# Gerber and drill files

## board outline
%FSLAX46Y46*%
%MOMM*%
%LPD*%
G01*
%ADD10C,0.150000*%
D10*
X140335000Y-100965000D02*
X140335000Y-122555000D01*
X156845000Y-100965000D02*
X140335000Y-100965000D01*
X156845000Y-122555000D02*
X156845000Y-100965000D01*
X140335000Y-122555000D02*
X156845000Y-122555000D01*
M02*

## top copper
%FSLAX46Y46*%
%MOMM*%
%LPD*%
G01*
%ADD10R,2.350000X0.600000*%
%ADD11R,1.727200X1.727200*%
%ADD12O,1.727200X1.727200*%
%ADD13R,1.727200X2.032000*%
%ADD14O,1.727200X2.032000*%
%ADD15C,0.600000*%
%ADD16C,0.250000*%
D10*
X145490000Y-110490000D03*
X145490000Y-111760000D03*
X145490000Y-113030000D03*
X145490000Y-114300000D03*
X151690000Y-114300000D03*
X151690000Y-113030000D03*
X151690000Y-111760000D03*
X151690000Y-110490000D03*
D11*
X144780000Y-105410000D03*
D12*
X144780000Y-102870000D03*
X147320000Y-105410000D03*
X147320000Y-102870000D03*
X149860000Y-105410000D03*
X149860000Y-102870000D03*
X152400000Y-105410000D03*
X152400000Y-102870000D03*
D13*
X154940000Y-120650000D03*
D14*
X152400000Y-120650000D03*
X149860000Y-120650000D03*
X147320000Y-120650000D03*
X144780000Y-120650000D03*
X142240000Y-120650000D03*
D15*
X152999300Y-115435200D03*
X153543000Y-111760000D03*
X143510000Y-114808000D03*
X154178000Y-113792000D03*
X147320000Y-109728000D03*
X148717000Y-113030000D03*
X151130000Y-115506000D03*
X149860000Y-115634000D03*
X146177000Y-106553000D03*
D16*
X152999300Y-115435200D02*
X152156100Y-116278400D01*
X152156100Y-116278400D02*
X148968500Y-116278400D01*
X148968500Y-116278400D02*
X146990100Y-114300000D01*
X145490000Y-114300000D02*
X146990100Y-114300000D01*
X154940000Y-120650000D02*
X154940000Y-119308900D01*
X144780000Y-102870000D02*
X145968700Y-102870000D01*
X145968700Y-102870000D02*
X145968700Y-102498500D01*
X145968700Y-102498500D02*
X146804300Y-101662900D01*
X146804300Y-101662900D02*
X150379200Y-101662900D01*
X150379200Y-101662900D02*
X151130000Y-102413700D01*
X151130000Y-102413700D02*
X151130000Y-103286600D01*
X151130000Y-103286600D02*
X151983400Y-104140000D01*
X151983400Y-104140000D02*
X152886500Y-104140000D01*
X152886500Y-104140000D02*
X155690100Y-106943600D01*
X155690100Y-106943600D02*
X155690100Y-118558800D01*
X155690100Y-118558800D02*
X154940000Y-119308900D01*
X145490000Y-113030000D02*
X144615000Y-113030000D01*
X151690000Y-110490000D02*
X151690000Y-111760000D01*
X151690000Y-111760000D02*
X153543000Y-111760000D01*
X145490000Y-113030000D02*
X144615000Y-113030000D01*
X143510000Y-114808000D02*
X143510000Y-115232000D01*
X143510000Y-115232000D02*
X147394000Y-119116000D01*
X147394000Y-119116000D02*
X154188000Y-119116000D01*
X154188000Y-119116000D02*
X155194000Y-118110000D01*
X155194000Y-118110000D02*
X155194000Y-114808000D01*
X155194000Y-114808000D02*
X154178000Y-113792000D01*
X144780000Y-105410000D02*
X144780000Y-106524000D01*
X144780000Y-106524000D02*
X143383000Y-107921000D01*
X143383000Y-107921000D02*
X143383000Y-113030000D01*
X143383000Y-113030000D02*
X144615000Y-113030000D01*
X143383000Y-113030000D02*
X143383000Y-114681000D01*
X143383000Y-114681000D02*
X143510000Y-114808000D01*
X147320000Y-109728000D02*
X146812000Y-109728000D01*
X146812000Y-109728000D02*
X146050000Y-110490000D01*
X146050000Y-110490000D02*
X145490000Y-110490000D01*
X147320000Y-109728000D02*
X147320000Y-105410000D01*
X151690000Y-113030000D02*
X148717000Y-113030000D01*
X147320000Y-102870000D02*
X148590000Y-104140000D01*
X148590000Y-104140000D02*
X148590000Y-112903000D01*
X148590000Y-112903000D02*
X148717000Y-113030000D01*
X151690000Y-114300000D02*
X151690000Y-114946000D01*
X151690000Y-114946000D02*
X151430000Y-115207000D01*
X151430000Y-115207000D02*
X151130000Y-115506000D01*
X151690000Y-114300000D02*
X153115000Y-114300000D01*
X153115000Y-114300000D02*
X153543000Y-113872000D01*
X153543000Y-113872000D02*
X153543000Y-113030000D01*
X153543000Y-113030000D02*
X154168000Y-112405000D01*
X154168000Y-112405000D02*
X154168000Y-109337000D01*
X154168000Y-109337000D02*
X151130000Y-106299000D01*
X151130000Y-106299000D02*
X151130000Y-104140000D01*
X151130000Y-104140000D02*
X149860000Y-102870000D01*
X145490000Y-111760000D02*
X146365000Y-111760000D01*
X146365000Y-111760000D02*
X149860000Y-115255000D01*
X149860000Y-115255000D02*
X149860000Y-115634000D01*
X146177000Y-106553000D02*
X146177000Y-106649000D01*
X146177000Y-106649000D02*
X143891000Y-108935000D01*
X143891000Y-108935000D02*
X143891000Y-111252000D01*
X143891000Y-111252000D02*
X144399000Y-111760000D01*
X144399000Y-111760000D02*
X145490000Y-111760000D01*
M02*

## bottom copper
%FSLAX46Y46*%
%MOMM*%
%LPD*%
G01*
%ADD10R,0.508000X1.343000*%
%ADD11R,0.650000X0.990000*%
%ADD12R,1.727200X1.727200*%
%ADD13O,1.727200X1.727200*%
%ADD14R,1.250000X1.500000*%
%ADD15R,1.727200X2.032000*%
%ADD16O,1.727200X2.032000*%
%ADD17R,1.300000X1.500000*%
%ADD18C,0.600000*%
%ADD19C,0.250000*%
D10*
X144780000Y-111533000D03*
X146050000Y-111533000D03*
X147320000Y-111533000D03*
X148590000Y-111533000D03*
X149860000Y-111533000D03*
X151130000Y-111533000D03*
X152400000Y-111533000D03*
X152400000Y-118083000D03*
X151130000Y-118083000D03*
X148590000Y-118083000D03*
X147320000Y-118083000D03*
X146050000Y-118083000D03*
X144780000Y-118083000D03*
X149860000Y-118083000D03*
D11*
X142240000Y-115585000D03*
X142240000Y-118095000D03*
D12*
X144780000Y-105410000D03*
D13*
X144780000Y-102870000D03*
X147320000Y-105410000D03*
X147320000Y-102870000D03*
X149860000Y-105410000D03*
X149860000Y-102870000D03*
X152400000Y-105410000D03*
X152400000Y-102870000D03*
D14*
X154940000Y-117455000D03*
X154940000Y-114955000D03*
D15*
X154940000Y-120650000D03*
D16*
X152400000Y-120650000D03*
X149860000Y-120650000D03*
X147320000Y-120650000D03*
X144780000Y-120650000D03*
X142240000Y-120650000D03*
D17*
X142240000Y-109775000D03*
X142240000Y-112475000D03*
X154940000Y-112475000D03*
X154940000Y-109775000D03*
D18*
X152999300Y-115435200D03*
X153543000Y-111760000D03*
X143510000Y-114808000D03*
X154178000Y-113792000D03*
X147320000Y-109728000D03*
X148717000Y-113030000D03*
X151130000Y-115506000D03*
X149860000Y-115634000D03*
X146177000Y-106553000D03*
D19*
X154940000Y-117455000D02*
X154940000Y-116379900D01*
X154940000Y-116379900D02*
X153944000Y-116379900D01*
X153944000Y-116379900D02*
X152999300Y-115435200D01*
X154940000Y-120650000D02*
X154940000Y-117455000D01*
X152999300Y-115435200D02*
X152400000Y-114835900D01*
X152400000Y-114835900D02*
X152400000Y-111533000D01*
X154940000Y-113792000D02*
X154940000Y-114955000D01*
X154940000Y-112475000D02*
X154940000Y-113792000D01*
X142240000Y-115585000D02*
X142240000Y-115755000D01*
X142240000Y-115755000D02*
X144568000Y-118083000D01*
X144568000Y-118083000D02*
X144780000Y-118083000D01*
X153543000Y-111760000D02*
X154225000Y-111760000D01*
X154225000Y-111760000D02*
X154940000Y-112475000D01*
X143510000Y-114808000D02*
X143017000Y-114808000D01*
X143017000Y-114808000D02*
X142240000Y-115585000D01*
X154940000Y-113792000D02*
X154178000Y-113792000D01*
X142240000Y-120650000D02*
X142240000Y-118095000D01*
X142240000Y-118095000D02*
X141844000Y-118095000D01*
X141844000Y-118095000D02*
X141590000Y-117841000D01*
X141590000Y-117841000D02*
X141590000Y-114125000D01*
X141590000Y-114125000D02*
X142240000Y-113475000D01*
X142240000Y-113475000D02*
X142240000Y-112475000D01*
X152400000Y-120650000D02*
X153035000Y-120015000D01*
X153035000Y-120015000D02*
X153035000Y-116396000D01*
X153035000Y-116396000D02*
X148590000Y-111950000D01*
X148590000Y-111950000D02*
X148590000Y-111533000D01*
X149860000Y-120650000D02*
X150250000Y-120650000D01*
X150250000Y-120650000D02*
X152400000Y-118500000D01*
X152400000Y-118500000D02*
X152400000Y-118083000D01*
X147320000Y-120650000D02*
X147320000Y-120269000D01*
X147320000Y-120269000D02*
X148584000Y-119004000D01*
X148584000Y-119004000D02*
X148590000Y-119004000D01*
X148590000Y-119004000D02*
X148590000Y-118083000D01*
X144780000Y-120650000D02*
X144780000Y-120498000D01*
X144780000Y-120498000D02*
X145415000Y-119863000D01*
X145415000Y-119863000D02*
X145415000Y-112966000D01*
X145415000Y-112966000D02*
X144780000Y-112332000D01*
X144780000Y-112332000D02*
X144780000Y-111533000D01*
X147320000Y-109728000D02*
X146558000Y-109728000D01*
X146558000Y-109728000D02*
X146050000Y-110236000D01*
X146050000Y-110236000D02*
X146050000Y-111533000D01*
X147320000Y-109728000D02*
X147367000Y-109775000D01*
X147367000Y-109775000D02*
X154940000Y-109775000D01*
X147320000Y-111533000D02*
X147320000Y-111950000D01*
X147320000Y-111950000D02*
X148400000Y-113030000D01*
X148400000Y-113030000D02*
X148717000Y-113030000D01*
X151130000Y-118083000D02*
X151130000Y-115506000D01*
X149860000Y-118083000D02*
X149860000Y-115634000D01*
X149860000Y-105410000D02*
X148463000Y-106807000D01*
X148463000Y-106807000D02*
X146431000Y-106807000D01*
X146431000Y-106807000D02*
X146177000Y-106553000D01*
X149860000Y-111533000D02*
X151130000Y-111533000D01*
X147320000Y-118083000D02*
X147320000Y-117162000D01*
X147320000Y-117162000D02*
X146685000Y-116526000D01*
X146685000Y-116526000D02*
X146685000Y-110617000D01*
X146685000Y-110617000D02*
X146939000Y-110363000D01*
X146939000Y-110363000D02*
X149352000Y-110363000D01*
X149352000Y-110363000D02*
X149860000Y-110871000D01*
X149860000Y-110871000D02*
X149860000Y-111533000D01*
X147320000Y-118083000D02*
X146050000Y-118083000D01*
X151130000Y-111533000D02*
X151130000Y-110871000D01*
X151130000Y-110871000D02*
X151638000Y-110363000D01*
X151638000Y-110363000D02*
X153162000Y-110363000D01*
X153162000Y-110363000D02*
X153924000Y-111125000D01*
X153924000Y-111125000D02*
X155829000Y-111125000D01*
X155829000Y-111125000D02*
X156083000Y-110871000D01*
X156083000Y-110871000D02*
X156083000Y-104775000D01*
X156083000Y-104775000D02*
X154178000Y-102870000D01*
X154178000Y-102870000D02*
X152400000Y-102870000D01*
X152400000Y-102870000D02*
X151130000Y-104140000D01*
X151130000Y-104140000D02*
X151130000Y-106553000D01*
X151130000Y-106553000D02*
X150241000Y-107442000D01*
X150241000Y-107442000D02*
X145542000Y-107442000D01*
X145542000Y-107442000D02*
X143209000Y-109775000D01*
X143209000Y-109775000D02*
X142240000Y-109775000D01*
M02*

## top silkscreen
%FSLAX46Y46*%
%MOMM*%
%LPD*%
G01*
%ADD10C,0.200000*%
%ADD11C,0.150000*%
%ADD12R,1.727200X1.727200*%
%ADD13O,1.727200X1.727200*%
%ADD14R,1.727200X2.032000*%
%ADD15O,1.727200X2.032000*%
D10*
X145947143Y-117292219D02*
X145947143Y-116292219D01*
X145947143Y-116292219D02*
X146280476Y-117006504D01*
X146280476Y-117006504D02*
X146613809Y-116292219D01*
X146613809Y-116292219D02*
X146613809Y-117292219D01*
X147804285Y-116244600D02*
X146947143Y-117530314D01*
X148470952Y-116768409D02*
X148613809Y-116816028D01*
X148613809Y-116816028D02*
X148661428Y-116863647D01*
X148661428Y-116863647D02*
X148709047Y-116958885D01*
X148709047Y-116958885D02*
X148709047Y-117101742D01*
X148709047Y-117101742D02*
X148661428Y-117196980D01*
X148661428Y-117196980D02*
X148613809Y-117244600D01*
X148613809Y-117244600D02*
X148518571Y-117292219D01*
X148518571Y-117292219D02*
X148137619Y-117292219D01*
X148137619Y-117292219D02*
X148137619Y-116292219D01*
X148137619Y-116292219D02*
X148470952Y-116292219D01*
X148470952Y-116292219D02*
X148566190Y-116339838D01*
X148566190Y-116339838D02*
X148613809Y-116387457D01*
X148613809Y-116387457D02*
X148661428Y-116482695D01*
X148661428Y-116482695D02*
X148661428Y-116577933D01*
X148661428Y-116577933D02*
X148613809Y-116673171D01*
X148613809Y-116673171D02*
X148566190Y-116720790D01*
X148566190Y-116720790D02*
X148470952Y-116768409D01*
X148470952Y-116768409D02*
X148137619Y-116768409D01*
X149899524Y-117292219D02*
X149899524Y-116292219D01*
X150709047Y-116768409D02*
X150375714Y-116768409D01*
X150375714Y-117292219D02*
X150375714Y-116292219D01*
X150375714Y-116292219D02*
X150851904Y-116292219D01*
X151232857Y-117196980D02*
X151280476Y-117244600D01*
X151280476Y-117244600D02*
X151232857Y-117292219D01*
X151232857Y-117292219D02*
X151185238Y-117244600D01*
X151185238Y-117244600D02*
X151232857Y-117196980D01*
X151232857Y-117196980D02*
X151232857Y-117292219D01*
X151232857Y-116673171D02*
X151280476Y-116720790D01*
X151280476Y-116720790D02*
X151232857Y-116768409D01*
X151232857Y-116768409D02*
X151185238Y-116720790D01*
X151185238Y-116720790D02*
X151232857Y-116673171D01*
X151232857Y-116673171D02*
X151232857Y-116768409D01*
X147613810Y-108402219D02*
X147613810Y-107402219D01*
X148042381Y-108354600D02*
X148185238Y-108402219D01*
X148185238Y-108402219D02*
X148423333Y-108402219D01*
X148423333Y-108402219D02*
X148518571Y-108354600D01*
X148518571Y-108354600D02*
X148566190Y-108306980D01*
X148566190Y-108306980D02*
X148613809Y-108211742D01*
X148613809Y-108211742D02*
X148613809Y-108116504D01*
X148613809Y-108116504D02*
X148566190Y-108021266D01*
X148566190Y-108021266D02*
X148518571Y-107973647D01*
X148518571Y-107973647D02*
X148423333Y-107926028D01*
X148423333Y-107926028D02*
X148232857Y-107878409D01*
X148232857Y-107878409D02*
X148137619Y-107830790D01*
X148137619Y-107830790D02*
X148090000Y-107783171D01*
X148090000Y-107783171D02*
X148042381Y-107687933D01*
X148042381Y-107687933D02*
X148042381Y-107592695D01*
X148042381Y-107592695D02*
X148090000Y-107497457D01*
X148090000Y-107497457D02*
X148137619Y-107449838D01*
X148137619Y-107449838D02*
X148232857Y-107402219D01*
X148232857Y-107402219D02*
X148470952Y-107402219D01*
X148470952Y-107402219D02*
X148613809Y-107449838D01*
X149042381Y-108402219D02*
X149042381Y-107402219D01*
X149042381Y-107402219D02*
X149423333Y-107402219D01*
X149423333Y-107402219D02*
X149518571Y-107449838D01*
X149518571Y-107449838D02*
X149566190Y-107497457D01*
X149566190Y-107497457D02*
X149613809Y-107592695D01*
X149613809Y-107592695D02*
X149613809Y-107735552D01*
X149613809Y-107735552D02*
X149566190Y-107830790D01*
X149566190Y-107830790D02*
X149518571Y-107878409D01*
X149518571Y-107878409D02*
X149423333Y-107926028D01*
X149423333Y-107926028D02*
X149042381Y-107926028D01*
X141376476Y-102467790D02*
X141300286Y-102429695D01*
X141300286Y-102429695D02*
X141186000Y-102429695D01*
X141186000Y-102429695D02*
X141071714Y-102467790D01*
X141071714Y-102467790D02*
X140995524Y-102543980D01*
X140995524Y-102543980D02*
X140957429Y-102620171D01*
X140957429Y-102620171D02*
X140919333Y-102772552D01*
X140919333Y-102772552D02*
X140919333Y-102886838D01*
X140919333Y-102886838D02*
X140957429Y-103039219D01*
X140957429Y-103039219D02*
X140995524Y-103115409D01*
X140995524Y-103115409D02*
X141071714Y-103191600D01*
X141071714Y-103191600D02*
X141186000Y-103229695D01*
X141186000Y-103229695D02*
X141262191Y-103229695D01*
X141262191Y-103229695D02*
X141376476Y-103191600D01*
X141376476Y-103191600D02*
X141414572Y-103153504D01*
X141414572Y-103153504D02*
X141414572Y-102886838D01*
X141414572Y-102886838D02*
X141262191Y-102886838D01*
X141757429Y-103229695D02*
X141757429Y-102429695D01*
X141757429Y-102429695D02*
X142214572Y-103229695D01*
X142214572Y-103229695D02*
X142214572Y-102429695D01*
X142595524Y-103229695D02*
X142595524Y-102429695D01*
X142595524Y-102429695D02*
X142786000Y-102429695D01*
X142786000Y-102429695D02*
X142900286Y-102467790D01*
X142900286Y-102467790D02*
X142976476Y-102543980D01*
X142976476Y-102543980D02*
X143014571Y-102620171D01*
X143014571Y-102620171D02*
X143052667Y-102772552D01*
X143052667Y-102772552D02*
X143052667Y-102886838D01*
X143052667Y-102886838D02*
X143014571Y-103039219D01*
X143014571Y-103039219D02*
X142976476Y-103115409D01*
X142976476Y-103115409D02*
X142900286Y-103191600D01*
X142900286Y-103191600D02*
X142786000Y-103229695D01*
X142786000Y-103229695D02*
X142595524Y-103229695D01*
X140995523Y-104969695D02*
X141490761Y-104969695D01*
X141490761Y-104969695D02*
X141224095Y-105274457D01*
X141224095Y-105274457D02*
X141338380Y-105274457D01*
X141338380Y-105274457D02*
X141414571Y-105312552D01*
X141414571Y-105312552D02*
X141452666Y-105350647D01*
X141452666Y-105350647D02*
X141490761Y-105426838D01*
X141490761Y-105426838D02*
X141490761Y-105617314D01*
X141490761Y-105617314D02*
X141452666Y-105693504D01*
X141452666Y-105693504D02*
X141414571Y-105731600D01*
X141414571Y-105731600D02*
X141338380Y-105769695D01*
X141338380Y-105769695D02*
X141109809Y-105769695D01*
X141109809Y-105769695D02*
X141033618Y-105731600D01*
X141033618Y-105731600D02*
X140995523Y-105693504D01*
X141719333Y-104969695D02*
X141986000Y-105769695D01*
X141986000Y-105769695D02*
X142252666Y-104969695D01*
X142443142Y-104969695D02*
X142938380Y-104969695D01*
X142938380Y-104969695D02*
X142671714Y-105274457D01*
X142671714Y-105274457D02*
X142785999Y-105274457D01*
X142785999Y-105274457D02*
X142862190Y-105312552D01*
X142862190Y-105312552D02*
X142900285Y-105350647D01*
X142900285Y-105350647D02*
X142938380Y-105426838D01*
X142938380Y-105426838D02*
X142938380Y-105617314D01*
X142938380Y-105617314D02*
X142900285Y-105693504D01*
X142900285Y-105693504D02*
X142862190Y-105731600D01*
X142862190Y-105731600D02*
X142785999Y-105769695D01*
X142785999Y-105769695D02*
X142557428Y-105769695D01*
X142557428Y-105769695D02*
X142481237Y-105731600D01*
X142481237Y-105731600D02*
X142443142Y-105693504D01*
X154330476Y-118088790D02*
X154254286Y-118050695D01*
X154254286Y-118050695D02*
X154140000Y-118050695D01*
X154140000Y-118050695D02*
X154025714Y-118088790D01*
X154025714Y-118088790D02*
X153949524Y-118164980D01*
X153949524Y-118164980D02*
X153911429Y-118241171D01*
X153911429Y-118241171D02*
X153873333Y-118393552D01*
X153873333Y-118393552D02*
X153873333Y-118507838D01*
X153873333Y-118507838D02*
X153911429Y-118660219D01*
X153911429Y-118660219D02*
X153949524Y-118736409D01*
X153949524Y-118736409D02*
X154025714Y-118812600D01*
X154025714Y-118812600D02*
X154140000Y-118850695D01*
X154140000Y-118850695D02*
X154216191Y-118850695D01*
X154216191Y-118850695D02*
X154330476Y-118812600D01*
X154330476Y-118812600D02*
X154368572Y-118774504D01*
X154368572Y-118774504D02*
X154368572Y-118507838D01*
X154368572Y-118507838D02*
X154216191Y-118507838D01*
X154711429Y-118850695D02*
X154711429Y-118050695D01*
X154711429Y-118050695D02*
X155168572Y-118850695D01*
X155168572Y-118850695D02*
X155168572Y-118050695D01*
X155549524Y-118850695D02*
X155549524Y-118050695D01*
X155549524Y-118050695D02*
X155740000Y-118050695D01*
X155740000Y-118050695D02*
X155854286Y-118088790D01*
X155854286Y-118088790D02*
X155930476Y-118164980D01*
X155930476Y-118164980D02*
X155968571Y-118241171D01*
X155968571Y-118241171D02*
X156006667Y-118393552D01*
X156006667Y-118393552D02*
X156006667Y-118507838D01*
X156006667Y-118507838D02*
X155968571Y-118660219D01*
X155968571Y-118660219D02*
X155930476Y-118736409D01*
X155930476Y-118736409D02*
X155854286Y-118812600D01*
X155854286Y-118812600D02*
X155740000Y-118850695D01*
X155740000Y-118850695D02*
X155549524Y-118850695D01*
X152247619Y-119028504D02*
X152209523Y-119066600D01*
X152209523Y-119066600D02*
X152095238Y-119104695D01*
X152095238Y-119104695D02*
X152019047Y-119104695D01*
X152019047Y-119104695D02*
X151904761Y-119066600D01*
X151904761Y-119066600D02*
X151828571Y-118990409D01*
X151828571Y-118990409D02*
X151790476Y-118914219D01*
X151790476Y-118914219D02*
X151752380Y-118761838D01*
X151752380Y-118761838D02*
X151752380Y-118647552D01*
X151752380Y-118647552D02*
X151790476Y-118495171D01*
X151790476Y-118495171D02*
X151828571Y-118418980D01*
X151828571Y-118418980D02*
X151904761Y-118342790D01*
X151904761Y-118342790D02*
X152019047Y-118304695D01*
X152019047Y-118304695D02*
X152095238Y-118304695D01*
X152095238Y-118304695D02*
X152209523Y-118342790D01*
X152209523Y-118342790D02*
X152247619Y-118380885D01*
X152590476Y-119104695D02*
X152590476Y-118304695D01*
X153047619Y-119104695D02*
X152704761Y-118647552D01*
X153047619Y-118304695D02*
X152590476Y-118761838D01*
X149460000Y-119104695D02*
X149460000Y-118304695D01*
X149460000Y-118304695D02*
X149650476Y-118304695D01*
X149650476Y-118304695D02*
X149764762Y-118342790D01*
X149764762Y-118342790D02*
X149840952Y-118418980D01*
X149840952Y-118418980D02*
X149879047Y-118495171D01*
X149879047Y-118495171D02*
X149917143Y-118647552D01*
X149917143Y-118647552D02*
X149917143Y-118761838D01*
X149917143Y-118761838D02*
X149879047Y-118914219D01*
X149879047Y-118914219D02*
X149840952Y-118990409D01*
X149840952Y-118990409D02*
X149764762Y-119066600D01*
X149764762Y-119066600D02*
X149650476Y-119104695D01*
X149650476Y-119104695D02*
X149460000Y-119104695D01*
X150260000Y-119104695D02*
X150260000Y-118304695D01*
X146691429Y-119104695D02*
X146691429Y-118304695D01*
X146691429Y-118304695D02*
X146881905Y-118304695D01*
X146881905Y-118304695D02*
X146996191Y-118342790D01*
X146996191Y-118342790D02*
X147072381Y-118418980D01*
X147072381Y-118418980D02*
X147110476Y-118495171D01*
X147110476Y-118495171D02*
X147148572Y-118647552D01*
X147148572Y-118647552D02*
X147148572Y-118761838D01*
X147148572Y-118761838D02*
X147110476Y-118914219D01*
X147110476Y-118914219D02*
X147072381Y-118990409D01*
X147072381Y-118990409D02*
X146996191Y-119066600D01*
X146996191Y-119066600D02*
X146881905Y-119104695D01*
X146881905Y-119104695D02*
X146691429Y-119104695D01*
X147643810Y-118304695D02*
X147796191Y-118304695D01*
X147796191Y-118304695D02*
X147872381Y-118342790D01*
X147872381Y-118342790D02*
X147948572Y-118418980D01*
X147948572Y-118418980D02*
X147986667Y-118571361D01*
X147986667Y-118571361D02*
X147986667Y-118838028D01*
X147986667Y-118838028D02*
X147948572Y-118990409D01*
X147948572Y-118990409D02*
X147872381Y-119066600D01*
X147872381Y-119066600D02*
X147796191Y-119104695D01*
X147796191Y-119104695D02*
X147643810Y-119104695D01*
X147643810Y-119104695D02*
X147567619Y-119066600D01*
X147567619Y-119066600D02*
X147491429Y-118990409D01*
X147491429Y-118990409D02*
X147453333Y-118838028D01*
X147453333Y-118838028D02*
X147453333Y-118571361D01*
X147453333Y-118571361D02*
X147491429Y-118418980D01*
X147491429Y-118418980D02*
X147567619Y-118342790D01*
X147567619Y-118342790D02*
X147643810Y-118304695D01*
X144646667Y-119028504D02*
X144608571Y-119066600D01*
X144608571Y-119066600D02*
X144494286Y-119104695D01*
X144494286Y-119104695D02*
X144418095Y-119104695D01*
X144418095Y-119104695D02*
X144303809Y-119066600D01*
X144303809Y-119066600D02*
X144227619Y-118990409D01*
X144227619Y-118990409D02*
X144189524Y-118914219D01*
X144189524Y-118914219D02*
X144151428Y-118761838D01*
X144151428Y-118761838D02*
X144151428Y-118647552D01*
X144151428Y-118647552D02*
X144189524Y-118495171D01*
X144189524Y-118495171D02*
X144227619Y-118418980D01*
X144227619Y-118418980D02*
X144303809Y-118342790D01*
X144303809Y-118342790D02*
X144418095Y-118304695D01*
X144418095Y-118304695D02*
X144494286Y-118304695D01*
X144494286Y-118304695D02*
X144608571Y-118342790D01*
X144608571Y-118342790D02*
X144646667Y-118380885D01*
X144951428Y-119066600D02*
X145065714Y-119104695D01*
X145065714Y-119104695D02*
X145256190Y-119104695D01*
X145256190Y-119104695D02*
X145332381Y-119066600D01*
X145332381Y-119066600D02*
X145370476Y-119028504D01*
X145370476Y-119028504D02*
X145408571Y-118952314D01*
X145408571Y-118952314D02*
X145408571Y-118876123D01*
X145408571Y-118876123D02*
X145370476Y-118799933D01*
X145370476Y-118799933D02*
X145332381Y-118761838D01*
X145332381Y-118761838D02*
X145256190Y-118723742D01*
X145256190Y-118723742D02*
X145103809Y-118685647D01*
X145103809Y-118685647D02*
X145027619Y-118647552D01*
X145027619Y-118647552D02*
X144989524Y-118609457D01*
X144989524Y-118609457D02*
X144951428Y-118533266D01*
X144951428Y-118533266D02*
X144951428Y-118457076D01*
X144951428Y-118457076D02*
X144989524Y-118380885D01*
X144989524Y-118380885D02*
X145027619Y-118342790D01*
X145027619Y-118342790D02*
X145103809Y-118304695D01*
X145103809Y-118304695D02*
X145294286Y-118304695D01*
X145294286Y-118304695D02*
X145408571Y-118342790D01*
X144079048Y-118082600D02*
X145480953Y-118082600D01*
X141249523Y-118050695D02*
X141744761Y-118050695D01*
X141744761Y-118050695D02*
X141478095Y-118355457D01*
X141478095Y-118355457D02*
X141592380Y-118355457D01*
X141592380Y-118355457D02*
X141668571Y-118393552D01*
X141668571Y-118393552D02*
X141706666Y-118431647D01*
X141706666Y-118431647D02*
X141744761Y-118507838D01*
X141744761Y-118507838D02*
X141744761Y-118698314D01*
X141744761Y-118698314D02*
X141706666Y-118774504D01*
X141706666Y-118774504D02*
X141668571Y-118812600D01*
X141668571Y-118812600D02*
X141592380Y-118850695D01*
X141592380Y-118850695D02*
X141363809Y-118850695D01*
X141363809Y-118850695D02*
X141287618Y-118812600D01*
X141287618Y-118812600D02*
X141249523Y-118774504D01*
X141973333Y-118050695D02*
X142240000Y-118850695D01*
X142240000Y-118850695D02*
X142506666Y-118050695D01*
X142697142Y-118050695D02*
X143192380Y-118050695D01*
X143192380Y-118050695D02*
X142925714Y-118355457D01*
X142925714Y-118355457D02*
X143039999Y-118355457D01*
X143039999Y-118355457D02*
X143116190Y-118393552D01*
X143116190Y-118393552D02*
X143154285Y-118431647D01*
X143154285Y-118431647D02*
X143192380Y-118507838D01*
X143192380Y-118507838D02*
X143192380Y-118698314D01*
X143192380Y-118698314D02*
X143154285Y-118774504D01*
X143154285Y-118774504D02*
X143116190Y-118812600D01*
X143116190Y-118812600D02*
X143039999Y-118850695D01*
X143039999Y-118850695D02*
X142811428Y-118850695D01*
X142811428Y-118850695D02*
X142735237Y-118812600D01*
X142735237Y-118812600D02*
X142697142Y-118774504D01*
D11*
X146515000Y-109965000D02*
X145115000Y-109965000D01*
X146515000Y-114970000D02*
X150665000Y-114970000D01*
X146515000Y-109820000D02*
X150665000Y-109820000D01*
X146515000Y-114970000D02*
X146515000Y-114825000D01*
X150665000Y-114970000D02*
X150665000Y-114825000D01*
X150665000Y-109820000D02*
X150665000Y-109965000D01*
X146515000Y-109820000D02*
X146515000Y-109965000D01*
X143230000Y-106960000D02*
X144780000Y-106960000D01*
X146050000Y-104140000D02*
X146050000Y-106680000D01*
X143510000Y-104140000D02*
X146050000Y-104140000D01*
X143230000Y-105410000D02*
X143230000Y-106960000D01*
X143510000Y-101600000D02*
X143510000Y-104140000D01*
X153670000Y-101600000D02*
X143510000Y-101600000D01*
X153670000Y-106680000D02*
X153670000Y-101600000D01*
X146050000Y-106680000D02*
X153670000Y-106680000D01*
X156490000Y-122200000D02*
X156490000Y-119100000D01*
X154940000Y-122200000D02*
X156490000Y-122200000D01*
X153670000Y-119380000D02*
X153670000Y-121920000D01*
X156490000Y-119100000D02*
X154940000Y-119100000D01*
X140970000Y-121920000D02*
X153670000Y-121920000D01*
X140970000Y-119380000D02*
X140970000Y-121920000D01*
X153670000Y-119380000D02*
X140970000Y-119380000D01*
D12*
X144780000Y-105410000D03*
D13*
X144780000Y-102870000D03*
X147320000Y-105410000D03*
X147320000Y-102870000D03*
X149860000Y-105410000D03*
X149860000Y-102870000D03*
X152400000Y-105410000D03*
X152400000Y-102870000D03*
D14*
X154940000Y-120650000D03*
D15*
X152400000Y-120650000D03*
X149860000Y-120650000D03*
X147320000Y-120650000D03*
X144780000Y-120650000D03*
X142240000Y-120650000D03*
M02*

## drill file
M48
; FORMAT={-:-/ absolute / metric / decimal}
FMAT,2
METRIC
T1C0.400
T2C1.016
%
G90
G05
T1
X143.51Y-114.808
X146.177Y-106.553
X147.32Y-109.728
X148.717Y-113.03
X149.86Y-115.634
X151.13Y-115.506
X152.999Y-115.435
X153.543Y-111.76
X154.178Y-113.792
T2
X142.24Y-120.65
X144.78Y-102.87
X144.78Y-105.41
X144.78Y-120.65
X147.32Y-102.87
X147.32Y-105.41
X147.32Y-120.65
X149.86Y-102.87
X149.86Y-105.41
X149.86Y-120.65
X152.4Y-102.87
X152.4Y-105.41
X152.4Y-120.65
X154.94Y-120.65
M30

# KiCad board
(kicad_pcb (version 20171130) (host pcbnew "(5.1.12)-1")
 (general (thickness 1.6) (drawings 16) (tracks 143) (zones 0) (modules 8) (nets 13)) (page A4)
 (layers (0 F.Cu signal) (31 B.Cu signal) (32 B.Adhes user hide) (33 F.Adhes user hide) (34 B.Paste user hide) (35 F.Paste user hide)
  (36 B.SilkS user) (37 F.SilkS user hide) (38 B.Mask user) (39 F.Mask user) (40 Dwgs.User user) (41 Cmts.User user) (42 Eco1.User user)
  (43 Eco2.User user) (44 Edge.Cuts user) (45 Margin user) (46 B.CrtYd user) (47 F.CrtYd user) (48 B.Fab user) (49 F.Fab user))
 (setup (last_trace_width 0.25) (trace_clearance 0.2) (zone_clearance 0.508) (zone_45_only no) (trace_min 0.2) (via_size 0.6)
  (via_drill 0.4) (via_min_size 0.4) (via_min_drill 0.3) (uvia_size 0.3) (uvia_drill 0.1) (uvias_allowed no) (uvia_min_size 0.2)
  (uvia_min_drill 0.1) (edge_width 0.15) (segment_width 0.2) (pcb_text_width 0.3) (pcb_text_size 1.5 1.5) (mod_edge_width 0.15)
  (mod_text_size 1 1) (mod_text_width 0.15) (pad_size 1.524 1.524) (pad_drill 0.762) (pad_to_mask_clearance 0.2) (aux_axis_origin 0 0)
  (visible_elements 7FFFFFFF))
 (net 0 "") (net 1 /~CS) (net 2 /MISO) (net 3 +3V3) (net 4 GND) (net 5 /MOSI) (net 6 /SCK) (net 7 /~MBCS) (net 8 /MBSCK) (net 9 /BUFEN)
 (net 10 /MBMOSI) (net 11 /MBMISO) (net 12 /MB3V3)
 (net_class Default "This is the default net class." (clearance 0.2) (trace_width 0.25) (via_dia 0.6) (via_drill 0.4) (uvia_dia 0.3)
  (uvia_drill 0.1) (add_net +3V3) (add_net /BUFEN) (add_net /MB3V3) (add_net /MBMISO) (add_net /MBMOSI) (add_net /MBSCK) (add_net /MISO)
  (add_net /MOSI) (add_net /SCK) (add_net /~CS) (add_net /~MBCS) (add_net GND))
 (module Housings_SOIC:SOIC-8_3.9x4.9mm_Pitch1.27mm (layer F.Cu) (at 148.59 112.395)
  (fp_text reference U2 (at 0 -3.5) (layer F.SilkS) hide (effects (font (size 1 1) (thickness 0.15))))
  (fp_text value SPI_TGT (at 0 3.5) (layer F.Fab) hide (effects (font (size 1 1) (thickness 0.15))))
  (fp_line (start -2.075 -2.43) (end -3.475 -2.43) (layer F.SilkS) (width 0.15))
  (fp_line (start -2.075 2.575) (end 2.075 2.575) (layer F.SilkS) (width 0.15))
  (fp_line (start -2.075 -2.575) (end 2.075 -2.575) (layer F.SilkS) (width 0.15))
  (fp_line (start -2.075 2.575) (end -2.075 2.43) (layer F.SilkS) (width 0.15))
  (fp_line (start 2.075 2.575) (end 2.075 2.43) (layer F.SilkS) (width 0.15))
  (fp_line (start 2.075 -2.575) (end 2.075 -2.43) (layer F.SilkS) (width 0.15))
  (fp_line (start -2.075 -2.575) (end -2.075 -2.43) (layer F.SilkS) (width 0.15))
  (pad 1 smd rect (at -3.1 -1.905) (size 2.35 0.6) (layers F.Cu F.Paste F.Mask) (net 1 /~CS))
  (pad 2 smd rect (at -3.1 -0.635) (size 2.35 0.6) (layers F.Cu F.Paste F.Mask) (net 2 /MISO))
  (pad 3 smd rect (at -3.1 0.635) (size 2.35 0.6) (layers F.Cu F.Paste F.Mask) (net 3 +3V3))
  (pad 4 smd rect (at -3.1 1.905) (size 2.35 0.6) (layers F.Cu F.Paste F.Mask) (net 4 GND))
  (pad 5 smd rect (at 3.1 1.905) (size 2.35 0.6) (layers F.Cu F.Paste F.Mask) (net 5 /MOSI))
  (pad 6 smd rect (at 3.1 0.635) (size 2.35 0.6) (layers F.Cu F.Paste F.Mask) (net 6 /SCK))
  (pad 7 smd rect (at 3.1 -0.635) (size 2.35 0.6) (layers F.Cu F.Paste F.Mask) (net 3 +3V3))
  (pad 8 smd rect (at 3.1 -1.905) (size 2.35 0.6) (layers F.Cu F.Paste F.Mask) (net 3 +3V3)))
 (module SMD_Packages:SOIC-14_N (layer B.Cu) (at 148.59 114.935)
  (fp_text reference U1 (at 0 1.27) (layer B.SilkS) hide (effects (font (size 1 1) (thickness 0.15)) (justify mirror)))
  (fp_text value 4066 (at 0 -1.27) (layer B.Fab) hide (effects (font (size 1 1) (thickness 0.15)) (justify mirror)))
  (pad 1 smd rect (at -3.81 -3.402) (size 0.508 1.343) (layers B.Cu B.Paste B.Mask) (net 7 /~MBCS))
  (pad 2 smd rect (at -2.54 -3.402) (size 0.508 1.343) (layers B.Cu B.Paste B.Mask) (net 1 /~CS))
  (pad 3 smd rect (at -1.27 -3.402) (size 0.508 1.343) (layers B.Cu B.Paste B.Mask) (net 6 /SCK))
  (pad 4 smd rect (at 0 -3.402) (size 0.508 1.343) (layers B.Cu B.Paste B.Mask) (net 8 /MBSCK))
  (pad 5 smd rect (at 1.27 -3.402) (size 0.508 1.343) (layers B.Cu B.Paste B.Mask) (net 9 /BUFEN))
  (pad 6 smd rect (at 2.54 -3.402) (size 0.508 1.343) (layers B.Cu B.Paste B.Mask) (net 9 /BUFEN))
  (pad 7 smd rect (at 3.81 -3.402) (size 0.508 1.343) (layers B.Cu B.Paste B.Mask) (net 4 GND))
  (pad 8 smd rect (at 3.81 3.148) (size 0.508 1.343) (layers B.Cu B.Paste B.Mask) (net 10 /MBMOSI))
  (pad 9 smd rect (at 2.54 3.148) (size 0.508 1.343) (layers B.Cu B.Paste B.Mask) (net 5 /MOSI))
  (pad 11 smd rect (at 0 3.148) (size 0.508 1.343) (layers B.Cu B.Paste B.Mask) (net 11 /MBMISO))
  (pad 12 smd rect (at -1.27 3.148) (size 0.508 1.343) (layers B.Cu B.Paste B.Mask) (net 9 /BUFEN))
  (pad 13 smd rect (at -2.54 3.148) (size 0.508 1.343) (layers B.Cu B.Paste B.Mask) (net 9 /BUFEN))
  (pad 14 smd rect (at -3.81 3.148) (size 0.508 1.343) (layers B.Cu B.Paste B.Mask) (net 3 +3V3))
  (pad 10 smd rect (at 1.27 3.148 180) (size 0.508 1.343) (layers B.Cu B.Paste B.Mask) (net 2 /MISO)))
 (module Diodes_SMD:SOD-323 (layer B.Cu) (at 142.24 116.84 270)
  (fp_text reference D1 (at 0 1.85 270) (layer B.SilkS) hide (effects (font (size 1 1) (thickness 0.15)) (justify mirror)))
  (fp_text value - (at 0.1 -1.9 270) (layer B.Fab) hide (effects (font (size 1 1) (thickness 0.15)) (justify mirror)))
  (pad 1 smd rect (at -1.255 0 270) (size 0.99 0.65) (layers B.Cu B.Paste B.Mask) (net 3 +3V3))
  (pad 2 smd rect (at 1.255 0 270) (size 0.99 0.65) (layers B.Cu B.Paste B.Mask) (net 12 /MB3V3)))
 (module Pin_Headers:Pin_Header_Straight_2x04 (layer F.Cu) (at 144.78 105.41 90)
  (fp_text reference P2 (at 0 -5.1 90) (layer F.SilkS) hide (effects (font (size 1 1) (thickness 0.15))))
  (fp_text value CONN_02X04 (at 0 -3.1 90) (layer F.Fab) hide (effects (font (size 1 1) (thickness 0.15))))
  (fp_line (start -1.55 -1.55) (end -1.55 0) (layer F.SilkS) (width 0.15))
  (fp_line (start 1.27 1.27) (end -1.27 1.27) (layer F.SilkS) (width 0.15))
  (fp_line (start 1.27 -1.27) (end 1.27 1.27) (layer F.SilkS) (width 0.15))
  (fp_line (start 0 -1.55) (end -1.55 -1.55) (layer F.SilkS) (width 0.15))
  (fp_line (start 3.81 -1.27) (end 1.27 -1.27) (layer F.SilkS) (width 0.15))
  (fp_line (start 3.81 8.89) (end 3.81 -1.27) (layer F.SilkS) (width 0.15))
  (fp_line (start -1.27 8.89) (end 3.81 8.89) (layer F.SilkS) (width 0.15))
  (fp_line (start -1.27 1.27) (end -1.27 8.89) (layer F.SilkS) (width 0.15))
  (pad 1 thru_hole rect (at 0 0 90) (size 1.7272 1.7272) (drill 1.016) (layers *.Cu *.Mask F.SilkS) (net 3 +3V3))
  (pad 2 thru_hole oval (at 2.54 0 90) (size 1.7272 1.7272) (drill 1.016) (layers *.Cu *.Mask F.SilkS) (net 4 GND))
  (pad 3 thru_hole oval (at 0 2.54 90) (size 1.7272 1.7272) (drill 1.016) (layers *.Cu *.Mask F.SilkS) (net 1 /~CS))
  (pad 4 thru_hole oval (at 2.54 2.54 90) (size 1.7272 1.7272) (drill 1.016) (layers *.Cu *.Mask F.SilkS) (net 6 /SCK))
  (pad 5 thru_hole oval (at 0 5.08 90) (size 1.7272 1.7272) (drill 1.016) (layers *.Cu *.Mask F.SilkS) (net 2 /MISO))
  (pad 6 thru_hole oval (at 2.54 5.08 90) (size 1.7272 1.7272) (drill 1.016) (layers *.Cu *.Mask F.SilkS) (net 5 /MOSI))
  (pad 7 thru_hole oval (at 0 7.62 90) (size 1.7272 1.7272) (drill 1.016) (layers *.Cu *.Mask F.SilkS))
  (pad 8 thru_hole oval (at 2.54 7.62 90) (size 1.7272 1.7272) (drill 1.016) (layers *.Cu *.Mask F.SilkS) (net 9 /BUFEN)))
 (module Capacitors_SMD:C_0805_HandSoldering (layer B.Cu) (at 154.94 116.205 90)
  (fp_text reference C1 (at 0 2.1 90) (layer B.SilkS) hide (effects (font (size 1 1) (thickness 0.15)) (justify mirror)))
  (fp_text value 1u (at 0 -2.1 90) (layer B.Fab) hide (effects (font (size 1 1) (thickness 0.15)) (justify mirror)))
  (pad 1 smd rect (at -1.25 0 90) (size 1.5 1.25) (layers B.Cu B.Paste B.Mask) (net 4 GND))
  (pad 2 smd rect (at 1.25 0 90) (size 1.5 1.25) (layers B.Cu B.Paste B.Mask) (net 3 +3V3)))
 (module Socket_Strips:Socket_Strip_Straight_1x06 (layer F.Cu) (at 154.94 120.65 180)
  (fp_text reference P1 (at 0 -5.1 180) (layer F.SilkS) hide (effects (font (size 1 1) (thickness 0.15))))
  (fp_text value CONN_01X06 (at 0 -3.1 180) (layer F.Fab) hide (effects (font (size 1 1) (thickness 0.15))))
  (fp_line (start -1.55 -1.55) (end -1.55 1.55) (layer F.SilkS) (width 0.15))
  (fp_line (start 0 -1.55) (end -1.55 -1.55) (layer F.SilkS) (width 0.15))
  (fp_line (start 1.27 1.27) (end 1.27 -1.27) (layer F.SilkS) (width 0.15))
  (fp_line (start -1.55 1.55) (end 0 1.55) (layer F.SilkS) (width 0.15))
  (fp_line (start 13.97 -1.27) (end 1.27 -1.27) (layer F.SilkS) (width 0.15))
  (fp_line (start 13.97 1.27) (end 13.97 -1.27) (layer F.SilkS) (width 0.15))
  (fp_line (start 1.27 1.27) (end 13.97 1.27) (layer F.SilkS) (width 0.15))
  (pad 1 thru_hole rect (at 0 0 180) (size 1.7272 2.032) (drill 1.016) (layers *.Cu *.Mask F.SilkS) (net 4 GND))
  (pad 2 thru_hole oval (at 2.54 0 180) (size 1.7272 2.032) (drill 1.016) (layers *.Cu *.Mask F.SilkS) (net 8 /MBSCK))
  (pad 3 thru_hole oval (at 5.08 0 180) (size 1.7272 2.032) (drill 1.016) (layers *.Cu *.Mask F.SilkS) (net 10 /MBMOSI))
  (pad 4 thru_hole oval (at 7.62 0 180) (size 1.7272 2.032) (drill 1.016) (layers *.Cu *.Mask F.SilkS) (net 11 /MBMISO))
  (pad 5 thru_hole oval (at 10.16 0 180) (size 1.7272 2.032) (drill 1.016) (layers *.Cu *.Mask F.SilkS) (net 7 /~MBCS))
  (pad 6 thru_hole oval (at 12.7 0 180) (size 1.7272 2.032) (drill 1.016) (layers *.Cu *.Mask F.SilkS) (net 12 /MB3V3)))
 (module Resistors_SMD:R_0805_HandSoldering (layer B.Cu) (at 142.24 111.125 270)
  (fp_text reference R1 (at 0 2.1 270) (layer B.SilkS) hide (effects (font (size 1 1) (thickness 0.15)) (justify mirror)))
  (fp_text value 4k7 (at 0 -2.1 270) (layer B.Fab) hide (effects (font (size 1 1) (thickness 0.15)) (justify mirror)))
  (pad 1 smd rect (at -1.35 0 270) (size 1.5 1.3) (layers B.Cu B.Paste B.Mask) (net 9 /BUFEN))
  (pad 2 smd rect (at 1.35 0 270) (size 1.5 1.3) (layers B.Cu B.Paste B.Mask) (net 12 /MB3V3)))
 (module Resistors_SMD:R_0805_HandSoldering (layer B.Cu) (at 154.94 111.125 90)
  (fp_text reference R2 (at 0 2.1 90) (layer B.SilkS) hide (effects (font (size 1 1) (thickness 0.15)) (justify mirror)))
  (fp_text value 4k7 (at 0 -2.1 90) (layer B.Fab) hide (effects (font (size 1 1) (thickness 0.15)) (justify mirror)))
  (pad 1 smd rect (at -1.35 0 90) (size 1.5 1.3) (layers B.Cu B.Paste B.Mask) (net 3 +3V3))
  (pad 2 smd rect (at 1.35 0 90) (size 1.5 1.3) (layers B.Cu B.Paste B.Mask) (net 1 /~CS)))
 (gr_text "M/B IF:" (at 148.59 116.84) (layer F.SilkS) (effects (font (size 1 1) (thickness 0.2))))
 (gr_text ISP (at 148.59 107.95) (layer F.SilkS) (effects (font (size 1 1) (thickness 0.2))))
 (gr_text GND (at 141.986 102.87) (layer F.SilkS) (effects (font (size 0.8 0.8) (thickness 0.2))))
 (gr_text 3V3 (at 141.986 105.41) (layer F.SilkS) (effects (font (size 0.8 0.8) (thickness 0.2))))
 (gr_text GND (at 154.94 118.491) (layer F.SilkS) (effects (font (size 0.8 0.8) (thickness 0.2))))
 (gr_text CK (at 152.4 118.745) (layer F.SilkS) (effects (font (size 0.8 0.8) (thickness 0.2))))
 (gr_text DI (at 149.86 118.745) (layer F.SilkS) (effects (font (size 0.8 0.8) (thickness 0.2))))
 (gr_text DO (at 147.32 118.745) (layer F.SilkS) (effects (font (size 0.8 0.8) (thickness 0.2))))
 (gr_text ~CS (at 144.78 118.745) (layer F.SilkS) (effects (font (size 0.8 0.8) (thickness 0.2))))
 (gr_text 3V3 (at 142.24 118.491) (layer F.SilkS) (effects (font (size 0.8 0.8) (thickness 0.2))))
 (gr_line (start 140.335 100.965) (end 140.335 122.555) (layer Edge.Cuts) (width 0.15))
 (gr_line (start 156.845 100.965) (end 140.335 100.965) (layer Edge.Cuts) (width 0.15))
 (gr_line (start 156.845 122.555) (end 156.845 100.965) (layer Edge.Cuts) (width 0.15))
 (gr_line (start 140.335 122.555) (end 156.845 122.555) (angle 90) (layer Edge.Cuts) (width 0.15))
 (segment (start 154.94 117.455) (end 154.94 116.3799) (width 0.25) (layer B.Cu) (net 4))
 (segment (start 154.94 116.3799) (end 153.944 116.3799) (width 0.25) (layer B.Cu) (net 4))
 (segment (start 153.944 116.3799) (end 152.9993 115.4352) (width 0.25) (layer B.Cu) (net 4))
 (segment (start 154.94 120.65) (end 154.94 117.455) (width 0.25) (layer B.Cu) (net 4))
 (segment (start 152.9993 115.4352) (end 152.4 114.8359) (width 0.25) (layer B.Cu) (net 4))
 (segment (start 152.4 114.8359) (end 152.4 111.533) (width 0.25) (layer B.Cu) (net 4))
 (segment (start 152.9993 115.4352) (end 152.1561 116.2784) (width 0.25) (layer F.Cu) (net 4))
 (segment (start 152.1561 116.2784) (end 148.9685 116.2784) (width 0.25) (layer F.Cu) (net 4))
 (segment (start 148.9685 116.2784) (end 146.9901 114.3) (width 0.25) (layer F.Cu) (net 4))
 (segment (start 145.49 114.3) (end 146.9901 114.3) (width 0.25) (layer F.Cu) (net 4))
 (segment (start 154.94 120.65) (end 154.94 119.3089) (width 0.25) (layer F.Cu) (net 4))
 (segment (start 144.78 102.87) (end 145.9687 102.87) (width 0.25) (layer F.Cu) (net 4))
 (segment (start 145.9687 102.87) (end 145.9687 102.4985) (width 0.25) (layer F.Cu) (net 4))
 (segment (start 145.9687 102.4985) (end 146.8043 101.6629) (width 0.25) (layer F.Cu) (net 4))
 (segment (start 146.8043 101.6629) (end 150.3792 101.6629) (width 0.25) (layer F.Cu) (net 4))
 (segment (start 150.3792 101.6629) (end 151.13 102.4137) (width 0.25) (layer F.Cu) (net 4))
 (segment (start 151.13 102.4137) (end 151.13 103.2866) (width 0.25) (layer F.Cu) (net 4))
 (segment (start 151.13 103.2866) (end 151.9834 104.14) (width 0.25) (layer F.Cu) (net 4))
 (segment (start 151.9834 104.14) (end 152.8865 104.14) (width 0.25) (layer F.Cu) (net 4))
 (segment (start 152.8865 104.14) (end 155.6901 106.9436) (width 0.25) (layer F.Cu) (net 4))
 (segment (start 155.6901 106.9436) (end 155.6901 118.5588) (width 0.25) (layer F.Cu) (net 4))
 (segment (start 155.6901 118.5588) (end 154.94 119.3089) (width 0.25) (layer F.Cu) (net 4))
 (via (at 152.9993 115.4352) (size 0.6) (layers F.Cu B.Cu) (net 4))
 (segment (start 154.94 113.792) (end 154.94 114.955) (width 0.25) (layer B.Cu) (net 3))
 (segment (start 154.94 112.475) (end 154.94 113.792) (width 0.25) (layer B.Cu) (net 3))
 (segment (start 145.49 113.03) (end 144.615 113.03) (width 0.25) (layer F.Cu) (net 3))
 (segment (start 142.24 115.585) (end 142.24 115.755) (width 0.25) (layer B.Cu) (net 3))
 (segment (start 142.24 115.755) (end 144.568 118.083) (width 0.25) (layer B.Cu) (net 3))
 (segment (start 144.568 118.083) (end 144.78 118.083) (width 0.25) (layer B.Cu) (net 3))
 (segment (start 151.69 110.49) (end 151.69 111.76) (width 0.25) (layer F.Cu) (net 3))
 (segment (start 151.69 111.76) (end 153.543 111.76) (width 0.25) (layer F.Cu) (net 3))
 (segment (start 153.543 111.76) (end 154.225 111.76) (width 0.25) (layer B.Cu) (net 3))
 (segment (start 154.225 111.76) (end 154.94 112.475) (width 0.25) (layer B.Cu) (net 3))
 (segment (start 145.49 113.03) (end 144.615 113.03) (width 0.25) (layer F.Cu) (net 3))
 (segment (start 143.51 114.808) (end 143.017 114.808) (width 0.25) (layer B.Cu) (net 3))
 (segment (start 143.017 114.808) (end 142.24 115.585) (width 0.25) (layer B.Cu) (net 3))
 (segment (start 154.94 113.792) (end 154.178 113.792) (width 0.25) (layer B.Cu) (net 3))
 (segment (start 143.51 114.808) (end 143.51 115.232) (width 0.25) (layer F.Cu) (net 3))
 (segment (start 143.51 115.232) (end 147.394 119.116) (width 0.25) (layer F.Cu) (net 3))
 (segment (start 147.394 119.116) (end 154.188 119.116) (width 0.25) (layer F.Cu) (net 3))
 (segment (start 154.188 119.116) (end 155.194 118.11) (width 0.25) (layer F.Cu) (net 3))
 (segment (start 155.194 118.11) (end 155.194 114.808) (width 0.25) (layer F.Cu) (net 3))
 (segment (start 155.194 114.808) (end 154.178 113.792) (width 0.25) (layer F.Cu) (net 3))
 (segment (start 144.78 105.41) (end 144.78 106.524) (width 0.25) (layer F.Cu) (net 3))
 (segment (start 144.78 106.524) (end 143.383 107.921) (width 0.25) (layer F.Cu) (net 3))
 (segment (start 143.383 107.921) (end 143.383 113.03) (width 0.25) (layer F.Cu) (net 3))
 (segment (start 143.383 113.03) (end 144.615 113.03) (width 0.25) (layer F.Cu) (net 3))
 (segment (start 143.383 113.03) (end 143.383 114.681) (width 0.25) (layer F.Cu) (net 3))
 (segment (start 143.383 114.681) (end 143.51 114.808) (width 0.25) (layer F.Cu) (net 3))
 (via (at 153.543 111.76) (size 0.6) (layers F.Cu B.Cu) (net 3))
 (via (at 143.51 114.808) (size 0.6) (layers F.Cu B.Cu) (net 3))
 (via (at 154.178 113.792) (size 0.6) (layers F.Cu B.Cu) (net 3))
 (segment (start 142.24 120.65) (end 142.24 118.095) (width 0.25) (layer B.Cu) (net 12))
 (segment (start 142.24 118.095) (end 141.844 118.095) (width 0.25) (layer B.Cu) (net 12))
 (segment (start 141.844 118.095) (end 141.59 117.841) (width 0.25) (layer B.Cu) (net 12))
 (segment (start 141.59 117.841) (end 141.59 114.125) (width 0.25) (layer B.Cu) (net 12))
 (segment (start 141.59 114.125) (end 142.24 113.475) (width 0.25) (layer B.Cu) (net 12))
 (segment (start 142.24 113.475) (end 142.24 112.475) (width 0.25) (layer B.Cu) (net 12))
 (segment (start 152.4 120.65) (end 153.035 120.015) (width 0.25) (layer B.Cu) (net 8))
 (segment (start 153.035 120.015) (end 153.035 116.396) (width 0.25) (layer B.Cu) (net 8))
 (segment (start 153.035 116.396) (end 148.59 111.95) (width 0.25) (layer B.Cu) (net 8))
 (segment (start 148.59 111.95) (end 148.59 111.533) (width 0.25) (layer B.Cu) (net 8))
 (segment (start 149.86 120.65) (end 150.25 120.65) (width 0.25) (layer B.Cu) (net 10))
 (segment (start 150.25 120.65) (end 152.4 118.5) (width 0.25) (layer B.Cu) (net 10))
 (segment (start 152.4 118.5) (end 152.4 118.083) (width 0.25) (layer B.Cu) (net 10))
 (segment (start 147.32 120.65) (end 147.32 120.269) (width 0.25) (layer B.Cu) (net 11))
 (segment (start 147.32 120.269) (end 148.584 119.004) (width 0.25) (layer B.Cu) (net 11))
 (segment (start 148.584 119.004) (end 148.59 119.004) (width 0.25) (layer B.Cu) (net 11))
 (segment (start 148.59 119.004) (end 148.59 118.083) (width 0.25) (layer B.Cu) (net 11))
 (segment (start 144.78 120.65) (end 144.78 120.498) (width 0.25) (layer B.Cu) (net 7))
 (segment (start 144.78 120.498) (end 145.415 119.863) (width 0.25) (layer B.Cu) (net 7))
 (segment (start 145.415 119.863) (end 145.415 112.966) (width 0.25) (layer B.Cu) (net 7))
 (segment (start 145.415 112.966) (end 144.78 112.332) (width 0.25) (layer B.Cu) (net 7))
 (segment (start 144.78 112.332) (end 144.78 111.533) (width 0.25) (layer B.Cu) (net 7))
 (segment (start 147.32 109.728) (end 146.558 109.728) (width 0.25) (layer B.Cu) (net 1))
 (segment (start 146.558 109.728) (end 146.05 110.236) (width 0.25) (layer B.Cu) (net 1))
 (segment (start 146.05 110.236) (end 146.05 111.533) (width 0.25) (layer B.Cu) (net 1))
 (segment (start 147.32 109.728) (end 146.812 109.728) (width 0.25) (layer F.Cu) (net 1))
 (segment (start 146.812 109.728) (end 146.05 110.49) (width 0.25) (layer F.Cu) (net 1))
 (segment (start 146.05 110.49) (end 145.49 110.49) (width 0.25) (layer F.Cu) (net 1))
 (segment (start 147.32 109.728) (end 147.32 105.41) (width 0.25) (layer F.Cu) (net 1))
 (segment (start 147.32 109.728) (end 147.367 109.775) (width 0.25) (layer B.Cu) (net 1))
 (segment (start 147.367 109.775) (end 154.94 109.775) (width 0.25) (layer B.Cu) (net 1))
 (via (at 147.32 109.728) (size 0.6) (layers F.Cu B.Cu) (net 1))
 (segment (start 151.69 113.03) (end 148.717 113.03) (width 0.25) (layer F.Cu) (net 6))
 (segment (start 147.32 111.533) (end 147.32 111.95) (width 0.25) (layer B.Cu) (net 6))
 (segment (start 147.32 111.95) (end 148.4 113.03) (width 0.25) (layer B.Cu) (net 6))
 (segment (start 148.4 113.03) (end 148.717 113.03) (width 0.25) (layer B.Cu) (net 6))
 (segment (start 147.32 102.87) (end 148.59 104.14) (width 0.25) (layer F.Cu) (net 6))
 (segment (start 148.59 104.14) (end 148.59 112.903) (width 0.25) (layer F.Cu) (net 6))
 (segment (start 148.59 112.903) (end 148.717 113.03) (width 0.25) (layer F.Cu) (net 6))
 (via (at 148.717 113.03) (size 0.6) (layers F.Cu B.Cu) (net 6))
 (segment (start 151.13 118.083) (end 151.13 115.506) (width 0.25) (layer B.Cu) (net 5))
 (segment (start 151.69 114.3) (end 151.69 114.946) (width 0.25) (layer F.Cu) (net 5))
 (segment (start 151.69 114.946) (end 151.43 115.207) (width 0.25) (layer F.Cu) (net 5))
 (segment (start 151.43 115.207) (end 151.13 115.506) (width 0.25) (layer F.Cu) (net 5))
 (segment (start 151.69 114.3) (end 153.115 114.3) (width 0.25) (layer F.Cu) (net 5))
 (segment (start 153.115 114.3) (end 153.543 113.872) (width 0.25) (layer F.Cu) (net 5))
 (segment (start 153.543 113.872) (end 153.543 113.03) (width 0.25) (layer F.Cu) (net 5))
 (segment (start 153.543 113.03) (end 154.168 112.405) (width 0.25) (layer F.Cu) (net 5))
 (segment (start 154.168 112.405) (end 154.168 109.337) (width 0.25) (layer F.Cu) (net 5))
 (segment (start 154.168 109.337) (end 151.13 106.299) (width 0.25) (layer F.Cu) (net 5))
 (segment (start 151.13 106.299) (end 151.13 104.14) (width 0.25) (layer F.Cu) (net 5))
 (segment (start 151.13 104.14) (end 149.86 102.87) (width 0.25) (layer F.Cu) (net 5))
 (via (at 151.13 115.506) (size 0.6) (layers F.Cu B.Cu) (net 5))
 (segment (start 149.86 118.083) (end 149.86 115.634) (width 0.25) (layer B.Cu) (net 2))
 (segment (start 145.49 111.76) (end 146.365 111.76) (width 0.25) (layer F.Cu) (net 2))
 (segment (start 146.365 111.76) (end 149.86 115.255) (width 0.25) (layer F.Cu) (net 2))
 (segment (start 149.86 115.255) (end 149.86 115.634) (width 0.25) (layer F.Cu) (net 2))
 (segment (start 146.177 106.553) (end 146.177 106.649) (width 0.25) (layer F.Cu) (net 2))
 (segment (start 146.177 106.649) (end 143.891 108.935) (width 0.25) (layer F.Cu) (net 2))
 (segment (start 143.891 108.935) (end 143.891 111.252) (width 0.25) (layer F.Cu) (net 2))
 (segment (start 143.891 111.252) (end 144.399 111.76) (width 0.25) (layer F.Cu) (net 2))
 (segment (start 144.399 111.76) (end 145.49 111.76) (width 0.25) (layer F.Cu) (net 2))
 (segment (start 149.86 105.41) (end 148.463 106.807) (width 0.25) (layer B.Cu) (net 2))
 (segment (start 148.463 106.807) (end 146.431 106.807) (width 0.25) (layer B.Cu) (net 2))
 (segment (start 146.431 106.807) (end 146.177 106.553) (width 0.25) (layer B.Cu) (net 2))
 (via (at 149.86 115.634) (size 0.6) (layers F.Cu B.Cu) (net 2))
 (via (at 146.177 106.553) (size 0.6) (layers F.Cu B.Cu) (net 2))
 (segment (start 149.86 111.533) (end 151.13 111.533) (width 0.25) (layer B.Cu) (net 9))
 (segment (start 147.32 118.083) (end 147.32 117.162) (width 0.25) (layer B.Cu) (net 9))
 (segment (start 147.32 117.162) (end 146.685 116.526) (width 0.25) (layer B.Cu) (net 9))
 (segment (start 146.685 116.526) (end 146.685 110.617) (width 0.25) (layer B.Cu) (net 9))
 (segment (start 146.685 110.617) (end 146.939 110.363) (width 0.25) (layer B.Cu) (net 9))
 (segment (start 146.939 110.363) (end 149.352 110.363) (width 0.25) (layer B.Cu) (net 9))
 (segment (start 149.352 110.363) (end 149.86 110.871) (width 0.25) (layer B.Cu) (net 9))
 (segment (start 149.86 110.871) (end 149.86 111.533) (width 0.25) (layer B.Cu) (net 9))
 (segment (start 147.32 118.083) (end 146.05 118.083) (width 0.25) (layer B.Cu) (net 9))
 (segment (start 151.13 111.533) (end 151.13 110.871) (width 0.25) (layer B.Cu) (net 9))
 (segment (start 151.13 110.871) (end 151.638 110.363) (width 0.25) (layer B.Cu) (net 9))
 (segment (start 151.638 110.363) (end 153.162 110.363) (width 0.25) (layer B.Cu) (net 9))
 (segment (start 153.162 110.363) (end 153.924 111.125) (width 0.25) (layer B.Cu) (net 9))
 (segment (start 153.924 111.125) (end 155.829 111.125) (width 0.25) (layer B.Cu) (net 9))
 (segment (start 155.829 111.125) (end 156.083 110.871) (width 0.25) (layer B.Cu) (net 9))
 (segment (start 156.083 110.871) (end 156.083 104.775) (width 0.25) (layer B.Cu) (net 9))
 (segment (start 156.083 104.775) (end 154.178 102.87) (width 0.25) (layer B.Cu) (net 9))
 (segment (start 154.178 102.87) (end 152.4 102.87) (width 0.25) (layer B.Cu) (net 9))
 (segment (start 152.4 102.87) (end 151.13 104.14) (width 0.25) (layer B.Cu) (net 9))
 (segment (start 151.13 104.14) (end 151.13 106.553) (width 0.25) (layer B.Cu) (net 9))
 (segment (start 151.13 106.553) (end 150.241 107.442) (width 0.25) (layer B.Cu) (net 9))
 (segment (start 150.241 107.442) (end 145.542 107.442) (width 0.25) (layer B.Cu) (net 9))
 (segment (start 145.542 107.442) (end 143.209 109.775) (width 0.25) (layer B.Cu) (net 9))
 (segment (start 143.209 109.775) (end 142.24 109.775) (width 0.25) (layer B.Cu) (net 9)))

